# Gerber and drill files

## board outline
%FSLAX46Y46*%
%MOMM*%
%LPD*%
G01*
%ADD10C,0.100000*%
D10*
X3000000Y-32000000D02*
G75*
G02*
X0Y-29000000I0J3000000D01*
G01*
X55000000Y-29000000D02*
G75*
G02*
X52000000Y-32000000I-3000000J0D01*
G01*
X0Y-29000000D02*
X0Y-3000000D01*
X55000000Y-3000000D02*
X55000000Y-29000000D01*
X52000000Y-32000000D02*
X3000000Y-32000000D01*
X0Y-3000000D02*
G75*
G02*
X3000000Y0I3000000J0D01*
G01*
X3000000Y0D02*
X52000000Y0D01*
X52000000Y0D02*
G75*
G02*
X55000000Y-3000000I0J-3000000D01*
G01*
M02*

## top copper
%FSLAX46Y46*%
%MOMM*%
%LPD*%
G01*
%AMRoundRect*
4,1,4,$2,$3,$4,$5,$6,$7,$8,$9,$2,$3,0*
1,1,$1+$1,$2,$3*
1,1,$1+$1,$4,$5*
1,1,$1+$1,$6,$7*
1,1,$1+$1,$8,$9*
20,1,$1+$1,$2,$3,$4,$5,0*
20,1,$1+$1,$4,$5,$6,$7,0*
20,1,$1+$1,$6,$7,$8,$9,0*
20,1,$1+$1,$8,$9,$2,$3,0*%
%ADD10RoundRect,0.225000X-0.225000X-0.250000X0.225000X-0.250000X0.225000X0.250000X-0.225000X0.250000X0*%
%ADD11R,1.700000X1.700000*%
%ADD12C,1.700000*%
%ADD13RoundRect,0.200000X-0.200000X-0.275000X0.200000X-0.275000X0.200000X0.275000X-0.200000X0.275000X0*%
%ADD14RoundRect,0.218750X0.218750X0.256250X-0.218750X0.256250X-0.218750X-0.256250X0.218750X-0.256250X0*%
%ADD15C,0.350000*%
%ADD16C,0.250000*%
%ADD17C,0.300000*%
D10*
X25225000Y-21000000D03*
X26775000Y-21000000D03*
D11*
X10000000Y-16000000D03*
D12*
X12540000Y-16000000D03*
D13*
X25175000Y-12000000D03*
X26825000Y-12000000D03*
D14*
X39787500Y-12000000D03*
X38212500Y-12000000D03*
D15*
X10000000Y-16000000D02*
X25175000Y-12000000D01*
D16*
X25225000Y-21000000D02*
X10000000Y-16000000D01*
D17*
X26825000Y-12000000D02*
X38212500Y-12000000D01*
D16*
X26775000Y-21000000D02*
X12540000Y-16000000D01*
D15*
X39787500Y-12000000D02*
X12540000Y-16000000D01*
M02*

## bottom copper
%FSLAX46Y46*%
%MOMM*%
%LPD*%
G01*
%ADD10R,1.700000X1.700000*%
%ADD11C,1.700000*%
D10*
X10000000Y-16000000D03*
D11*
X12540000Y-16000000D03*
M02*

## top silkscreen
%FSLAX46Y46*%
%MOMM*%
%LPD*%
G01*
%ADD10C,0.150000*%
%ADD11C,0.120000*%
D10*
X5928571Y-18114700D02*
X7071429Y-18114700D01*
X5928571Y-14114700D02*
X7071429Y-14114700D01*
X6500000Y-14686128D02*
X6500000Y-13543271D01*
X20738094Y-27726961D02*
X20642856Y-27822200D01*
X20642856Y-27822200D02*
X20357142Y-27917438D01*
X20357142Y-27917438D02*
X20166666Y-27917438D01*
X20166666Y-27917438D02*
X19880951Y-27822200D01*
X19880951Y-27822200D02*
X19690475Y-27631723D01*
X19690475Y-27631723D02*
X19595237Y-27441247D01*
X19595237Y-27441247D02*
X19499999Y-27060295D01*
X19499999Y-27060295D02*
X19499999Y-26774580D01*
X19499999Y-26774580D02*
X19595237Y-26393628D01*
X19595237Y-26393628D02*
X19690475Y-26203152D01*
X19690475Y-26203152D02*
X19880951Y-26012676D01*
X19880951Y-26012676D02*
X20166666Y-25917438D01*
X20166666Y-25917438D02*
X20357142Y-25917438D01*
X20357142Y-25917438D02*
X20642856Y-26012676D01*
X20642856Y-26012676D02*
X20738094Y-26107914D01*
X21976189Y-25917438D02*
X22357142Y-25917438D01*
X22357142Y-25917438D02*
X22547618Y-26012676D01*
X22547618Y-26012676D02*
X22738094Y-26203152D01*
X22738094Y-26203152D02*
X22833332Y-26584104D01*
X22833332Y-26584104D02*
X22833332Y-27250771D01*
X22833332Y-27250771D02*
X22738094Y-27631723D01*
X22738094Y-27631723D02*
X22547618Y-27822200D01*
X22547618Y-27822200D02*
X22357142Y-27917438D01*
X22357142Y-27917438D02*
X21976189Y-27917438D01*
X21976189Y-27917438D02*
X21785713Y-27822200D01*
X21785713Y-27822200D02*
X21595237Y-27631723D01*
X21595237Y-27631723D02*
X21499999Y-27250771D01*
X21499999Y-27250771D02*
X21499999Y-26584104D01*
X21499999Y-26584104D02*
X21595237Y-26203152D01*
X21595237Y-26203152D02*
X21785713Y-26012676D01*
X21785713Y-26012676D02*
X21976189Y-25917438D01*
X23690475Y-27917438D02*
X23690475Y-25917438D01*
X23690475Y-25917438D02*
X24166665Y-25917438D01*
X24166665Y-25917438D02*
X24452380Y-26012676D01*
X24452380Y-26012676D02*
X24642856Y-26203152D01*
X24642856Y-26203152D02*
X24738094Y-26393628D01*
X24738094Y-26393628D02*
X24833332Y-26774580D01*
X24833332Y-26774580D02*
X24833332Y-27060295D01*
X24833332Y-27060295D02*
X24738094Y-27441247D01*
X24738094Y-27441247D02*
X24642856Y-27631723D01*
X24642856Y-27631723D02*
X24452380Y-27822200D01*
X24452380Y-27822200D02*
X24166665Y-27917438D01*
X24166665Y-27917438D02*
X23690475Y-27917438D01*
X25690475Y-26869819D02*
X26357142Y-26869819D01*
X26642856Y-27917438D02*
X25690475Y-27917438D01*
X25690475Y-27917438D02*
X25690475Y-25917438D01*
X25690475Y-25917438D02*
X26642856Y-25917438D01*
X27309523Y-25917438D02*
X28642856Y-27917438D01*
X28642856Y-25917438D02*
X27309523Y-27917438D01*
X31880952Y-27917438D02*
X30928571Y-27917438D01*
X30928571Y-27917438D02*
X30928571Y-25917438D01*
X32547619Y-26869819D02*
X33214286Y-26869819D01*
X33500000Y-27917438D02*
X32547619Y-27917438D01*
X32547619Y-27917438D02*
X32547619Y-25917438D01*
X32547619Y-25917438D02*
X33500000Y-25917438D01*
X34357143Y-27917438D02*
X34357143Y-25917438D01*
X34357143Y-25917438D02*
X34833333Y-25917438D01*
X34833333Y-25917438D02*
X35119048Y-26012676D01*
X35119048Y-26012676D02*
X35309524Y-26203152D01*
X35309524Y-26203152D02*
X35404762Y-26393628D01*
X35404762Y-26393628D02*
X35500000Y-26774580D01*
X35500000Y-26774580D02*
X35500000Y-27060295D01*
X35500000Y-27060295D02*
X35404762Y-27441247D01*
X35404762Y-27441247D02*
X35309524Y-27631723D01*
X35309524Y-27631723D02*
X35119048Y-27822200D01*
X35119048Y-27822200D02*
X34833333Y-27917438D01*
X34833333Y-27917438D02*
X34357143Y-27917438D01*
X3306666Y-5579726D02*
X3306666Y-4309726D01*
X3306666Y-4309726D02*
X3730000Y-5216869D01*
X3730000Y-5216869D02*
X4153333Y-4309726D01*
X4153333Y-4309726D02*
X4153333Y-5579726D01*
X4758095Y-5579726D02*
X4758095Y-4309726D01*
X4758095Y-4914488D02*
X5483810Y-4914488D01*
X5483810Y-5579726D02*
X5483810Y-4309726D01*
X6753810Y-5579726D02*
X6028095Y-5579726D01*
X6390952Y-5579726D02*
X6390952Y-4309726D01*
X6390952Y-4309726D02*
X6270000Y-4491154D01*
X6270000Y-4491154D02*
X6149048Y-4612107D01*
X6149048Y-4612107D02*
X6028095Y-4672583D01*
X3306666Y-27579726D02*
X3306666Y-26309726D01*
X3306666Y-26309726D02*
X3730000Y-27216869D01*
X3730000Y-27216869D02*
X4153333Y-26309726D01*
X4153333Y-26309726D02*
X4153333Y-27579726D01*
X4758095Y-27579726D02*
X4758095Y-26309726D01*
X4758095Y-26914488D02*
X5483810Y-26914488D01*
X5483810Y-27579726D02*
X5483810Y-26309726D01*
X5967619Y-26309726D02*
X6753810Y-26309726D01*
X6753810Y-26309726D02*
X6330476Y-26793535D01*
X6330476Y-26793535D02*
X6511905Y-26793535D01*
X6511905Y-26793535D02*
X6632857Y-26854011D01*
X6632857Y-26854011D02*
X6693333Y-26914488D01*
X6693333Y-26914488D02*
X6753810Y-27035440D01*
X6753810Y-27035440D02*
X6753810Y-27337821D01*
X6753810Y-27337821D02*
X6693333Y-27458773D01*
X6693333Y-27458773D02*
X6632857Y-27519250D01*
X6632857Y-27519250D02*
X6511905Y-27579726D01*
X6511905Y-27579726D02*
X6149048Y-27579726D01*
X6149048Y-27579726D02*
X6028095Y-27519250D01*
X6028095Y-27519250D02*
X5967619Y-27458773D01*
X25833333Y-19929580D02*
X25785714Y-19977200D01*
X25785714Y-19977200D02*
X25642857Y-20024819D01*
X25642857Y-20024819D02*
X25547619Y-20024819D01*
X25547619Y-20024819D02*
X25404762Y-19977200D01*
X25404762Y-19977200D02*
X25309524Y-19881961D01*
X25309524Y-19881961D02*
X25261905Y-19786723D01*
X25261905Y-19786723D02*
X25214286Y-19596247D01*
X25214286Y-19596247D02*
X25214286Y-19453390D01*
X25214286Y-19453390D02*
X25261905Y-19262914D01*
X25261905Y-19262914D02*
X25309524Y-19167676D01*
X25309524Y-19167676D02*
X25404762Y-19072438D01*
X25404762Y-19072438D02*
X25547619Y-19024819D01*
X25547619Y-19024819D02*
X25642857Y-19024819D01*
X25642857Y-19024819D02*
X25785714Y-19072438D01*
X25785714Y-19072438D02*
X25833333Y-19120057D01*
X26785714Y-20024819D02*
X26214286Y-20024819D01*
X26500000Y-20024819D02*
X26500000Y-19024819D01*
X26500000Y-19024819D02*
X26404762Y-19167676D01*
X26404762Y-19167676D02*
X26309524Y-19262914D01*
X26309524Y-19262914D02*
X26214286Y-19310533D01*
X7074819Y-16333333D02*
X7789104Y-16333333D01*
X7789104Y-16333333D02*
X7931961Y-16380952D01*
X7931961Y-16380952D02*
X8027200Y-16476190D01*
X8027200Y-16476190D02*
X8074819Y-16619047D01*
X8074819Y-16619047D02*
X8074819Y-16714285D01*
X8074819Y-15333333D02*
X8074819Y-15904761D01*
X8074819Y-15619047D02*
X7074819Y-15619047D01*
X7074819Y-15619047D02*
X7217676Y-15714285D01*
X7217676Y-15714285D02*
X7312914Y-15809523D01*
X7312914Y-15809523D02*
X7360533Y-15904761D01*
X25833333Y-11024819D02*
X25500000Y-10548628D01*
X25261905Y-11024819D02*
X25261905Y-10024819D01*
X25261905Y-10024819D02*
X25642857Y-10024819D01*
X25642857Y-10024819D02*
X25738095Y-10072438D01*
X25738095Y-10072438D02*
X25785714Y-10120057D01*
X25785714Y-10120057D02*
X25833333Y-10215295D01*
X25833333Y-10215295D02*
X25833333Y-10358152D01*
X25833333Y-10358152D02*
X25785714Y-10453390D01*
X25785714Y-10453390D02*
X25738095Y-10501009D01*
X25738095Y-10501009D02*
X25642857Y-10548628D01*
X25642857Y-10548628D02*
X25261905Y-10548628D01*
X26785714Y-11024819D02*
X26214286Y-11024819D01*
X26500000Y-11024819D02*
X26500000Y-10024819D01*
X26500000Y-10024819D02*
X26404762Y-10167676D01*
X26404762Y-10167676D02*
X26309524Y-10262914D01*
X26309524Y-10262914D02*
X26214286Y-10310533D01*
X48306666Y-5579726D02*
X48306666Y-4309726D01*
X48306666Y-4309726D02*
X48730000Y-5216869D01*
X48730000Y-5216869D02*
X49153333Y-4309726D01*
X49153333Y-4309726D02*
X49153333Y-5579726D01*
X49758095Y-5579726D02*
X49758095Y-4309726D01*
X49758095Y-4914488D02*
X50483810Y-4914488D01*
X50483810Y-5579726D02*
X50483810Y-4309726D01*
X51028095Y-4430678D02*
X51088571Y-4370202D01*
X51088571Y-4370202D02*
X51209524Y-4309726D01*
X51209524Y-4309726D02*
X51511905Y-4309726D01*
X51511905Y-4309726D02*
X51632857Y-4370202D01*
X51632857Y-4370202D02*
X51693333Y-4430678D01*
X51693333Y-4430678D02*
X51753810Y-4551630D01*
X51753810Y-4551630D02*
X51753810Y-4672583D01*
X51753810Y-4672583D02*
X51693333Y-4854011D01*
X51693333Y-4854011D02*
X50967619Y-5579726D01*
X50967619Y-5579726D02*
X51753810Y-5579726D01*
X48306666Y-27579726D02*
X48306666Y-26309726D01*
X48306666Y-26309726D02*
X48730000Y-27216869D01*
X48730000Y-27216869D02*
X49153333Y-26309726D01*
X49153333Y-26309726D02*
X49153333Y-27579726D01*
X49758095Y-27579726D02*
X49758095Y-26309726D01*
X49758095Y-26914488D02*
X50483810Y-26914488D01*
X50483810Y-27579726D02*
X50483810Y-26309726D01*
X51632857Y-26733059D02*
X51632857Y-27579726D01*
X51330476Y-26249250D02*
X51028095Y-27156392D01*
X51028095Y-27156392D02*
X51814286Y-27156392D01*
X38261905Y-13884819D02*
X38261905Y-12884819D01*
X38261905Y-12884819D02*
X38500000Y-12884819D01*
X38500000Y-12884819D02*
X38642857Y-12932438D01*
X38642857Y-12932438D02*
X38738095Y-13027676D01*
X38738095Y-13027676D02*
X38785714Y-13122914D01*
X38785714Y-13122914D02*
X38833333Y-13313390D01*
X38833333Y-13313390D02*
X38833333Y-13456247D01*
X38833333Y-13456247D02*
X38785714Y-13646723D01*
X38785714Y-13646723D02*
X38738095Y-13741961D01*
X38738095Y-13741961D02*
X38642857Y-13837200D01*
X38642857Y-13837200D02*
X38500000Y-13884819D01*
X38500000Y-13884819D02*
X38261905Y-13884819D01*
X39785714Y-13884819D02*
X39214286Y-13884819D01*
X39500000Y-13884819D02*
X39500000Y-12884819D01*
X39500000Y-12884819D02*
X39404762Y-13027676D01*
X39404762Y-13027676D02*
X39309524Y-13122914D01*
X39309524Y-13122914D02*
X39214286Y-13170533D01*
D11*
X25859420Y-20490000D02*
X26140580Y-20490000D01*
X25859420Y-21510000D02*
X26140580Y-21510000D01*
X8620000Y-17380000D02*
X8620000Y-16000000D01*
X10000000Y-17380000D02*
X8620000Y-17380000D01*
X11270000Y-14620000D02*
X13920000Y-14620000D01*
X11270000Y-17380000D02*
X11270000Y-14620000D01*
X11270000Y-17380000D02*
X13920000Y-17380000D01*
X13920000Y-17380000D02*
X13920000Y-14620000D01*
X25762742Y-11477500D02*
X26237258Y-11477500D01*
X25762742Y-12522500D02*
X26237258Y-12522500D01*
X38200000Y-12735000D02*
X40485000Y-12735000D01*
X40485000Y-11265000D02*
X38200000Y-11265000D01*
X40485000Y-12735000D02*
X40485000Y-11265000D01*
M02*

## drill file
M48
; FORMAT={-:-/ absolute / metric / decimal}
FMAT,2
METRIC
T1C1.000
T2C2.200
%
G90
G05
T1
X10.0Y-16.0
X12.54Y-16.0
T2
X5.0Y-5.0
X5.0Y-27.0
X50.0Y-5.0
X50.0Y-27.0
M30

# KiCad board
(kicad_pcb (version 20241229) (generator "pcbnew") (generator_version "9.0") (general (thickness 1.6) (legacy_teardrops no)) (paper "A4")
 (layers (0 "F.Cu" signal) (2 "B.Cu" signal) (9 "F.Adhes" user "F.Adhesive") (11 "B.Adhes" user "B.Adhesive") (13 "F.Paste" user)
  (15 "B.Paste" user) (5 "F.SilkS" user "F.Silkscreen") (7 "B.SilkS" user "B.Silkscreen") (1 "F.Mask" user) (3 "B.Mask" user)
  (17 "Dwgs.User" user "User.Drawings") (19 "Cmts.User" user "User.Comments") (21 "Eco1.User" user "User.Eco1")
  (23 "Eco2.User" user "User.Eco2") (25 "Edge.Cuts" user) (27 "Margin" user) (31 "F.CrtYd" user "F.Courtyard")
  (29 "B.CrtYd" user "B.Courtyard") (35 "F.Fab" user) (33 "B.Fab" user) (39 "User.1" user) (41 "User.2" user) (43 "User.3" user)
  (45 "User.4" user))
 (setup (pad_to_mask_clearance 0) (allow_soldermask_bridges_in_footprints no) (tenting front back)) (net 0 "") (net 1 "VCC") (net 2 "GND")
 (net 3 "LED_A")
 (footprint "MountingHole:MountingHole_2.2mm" (layer "F.Cu") (at 5 5)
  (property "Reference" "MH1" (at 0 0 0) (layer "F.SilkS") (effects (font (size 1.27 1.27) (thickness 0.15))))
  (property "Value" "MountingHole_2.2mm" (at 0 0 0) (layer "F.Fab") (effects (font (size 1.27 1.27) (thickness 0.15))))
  (pad "" np_thru_hole circle (at 0 0) (size 3.2 3.2) (drill 2.2) (layers "*.Mask")))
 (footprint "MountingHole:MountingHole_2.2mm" (layer "F.Cu") (at 5 27)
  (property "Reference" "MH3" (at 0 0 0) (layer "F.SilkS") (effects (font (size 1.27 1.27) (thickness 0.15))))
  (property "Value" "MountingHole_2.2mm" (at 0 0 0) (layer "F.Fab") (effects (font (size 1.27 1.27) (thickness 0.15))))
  (pad "" np_thru_hole circle (at 0 0) (size 3.2 3.2) (drill 2.2) (layers "*.Mask")))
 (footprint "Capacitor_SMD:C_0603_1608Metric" (layer "F.Cu") (at 26 21)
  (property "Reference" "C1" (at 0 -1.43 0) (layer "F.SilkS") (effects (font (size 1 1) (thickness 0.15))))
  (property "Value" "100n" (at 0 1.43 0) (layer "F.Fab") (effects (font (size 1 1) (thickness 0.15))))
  (fp_line (start -0.14058 -0.51) (end 0.14058 -0.51) (stroke (width 0.12) (type solid)) (layer "F.SilkS"))
  (fp_line (start -0.14058 0.51) (end 0.14058 0.51) (stroke (width 0.12) (type solid)) (layer "F.SilkS"))
  (pad "1" smd roundrect (at -0.775 0) (size 0.9 0.95) (layers "F.Cu" "F.Mask" "F.Paste") (roundrect_rratio 0.25) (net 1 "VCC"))
  (pad "2" smd roundrect (at 0.775 0) (size 0.9 0.95) (layers "F.Cu" "F.Mask" "F.Paste") (roundrect_rratio 0.25) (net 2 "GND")))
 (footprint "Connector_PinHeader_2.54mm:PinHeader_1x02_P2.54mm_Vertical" (layer "F.Cu") (at 10 16 90)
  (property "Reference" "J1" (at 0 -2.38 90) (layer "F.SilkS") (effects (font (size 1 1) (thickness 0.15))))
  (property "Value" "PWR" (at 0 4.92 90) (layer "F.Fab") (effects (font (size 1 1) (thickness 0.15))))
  (fp_line (start -1.38 -1.38) (end 0 -1.38) (stroke (width 0.12) (type solid)) (layer "F.SilkS"))
  (fp_line (start -1.38 0) (end -1.38 -1.38) (stroke (width 0.12) (type solid)) (layer "F.SilkS"))
  (fp_line (start 1.38 1.27) (end 1.38 3.92) (stroke (width 0.12) (type solid)) (layer "F.SilkS"))
  (fp_line (start -1.38 1.27) (end 1.38 1.27) (stroke (width 0.12) (type solid)) (layer "F.SilkS"))
  (fp_line (start -1.38 1.27) (end -1.38 3.92) (stroke (width 0.12) (type solid)) (layer "F.SilkS"))
  (fp_line (start -1.38 3.92) (end 1.38 3.92) (stroke (width 0.12) (type solid)) (layer "F.SilkS"))
  (pad "1" thru_hole rect (at 0 0 90) (size 1.7 1.7) (drill 1) (layers "*.Cu" "*.Mask") (remove_unused_layers no) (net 1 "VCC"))
  (pad "2" thru_hole circle (at 0 2.54 90) (size 1.7 1.7) (drill 1) (layers "*.Cu" "*.Mask") (remove_unused_layers no) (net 2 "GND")))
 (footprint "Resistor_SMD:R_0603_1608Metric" (layer "F.Cu") (at 26 12)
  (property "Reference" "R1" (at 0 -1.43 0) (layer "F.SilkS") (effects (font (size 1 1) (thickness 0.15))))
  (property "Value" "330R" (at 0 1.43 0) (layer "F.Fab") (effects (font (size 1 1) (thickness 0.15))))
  (fp_line (start -0.237258 -0.5225) (end 0.237258 -0.5225) (stroke (width 0.12) (type solid)) (layer "F.SilkS"))
  (fp_line (start -0.237258 0.5225) (end 0.237258 0.5225) (stroke (width 0.12) (type solid)) (layer "F.SilkS"))
  (pad "1" smd roundrect (at -0.825 0) (size 0.8 0.95) (layers "F.Cu" "F.Mask" "F.Paste") (roundrect_rratio 0.25) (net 1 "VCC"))
  (pad "2" smd roundrect (at 0.825 0) (size 0.8 0.95) (layers "F.Cu" "F.Mask" "F.Paste") (roundrect_rratio 0.25) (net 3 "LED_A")))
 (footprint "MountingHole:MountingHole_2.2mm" (layer "F.Cu") (at 50 5)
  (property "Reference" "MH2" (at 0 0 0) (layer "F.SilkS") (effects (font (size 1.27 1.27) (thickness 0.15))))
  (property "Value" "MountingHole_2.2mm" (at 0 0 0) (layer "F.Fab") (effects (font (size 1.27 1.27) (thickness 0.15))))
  (pad "" np_thru_hole circle (at 0 0) (size 3.2 3.2) (drill 2.2) (layers "*.Mask")))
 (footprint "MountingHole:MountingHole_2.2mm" (layer "F.Cu") (at 50 27)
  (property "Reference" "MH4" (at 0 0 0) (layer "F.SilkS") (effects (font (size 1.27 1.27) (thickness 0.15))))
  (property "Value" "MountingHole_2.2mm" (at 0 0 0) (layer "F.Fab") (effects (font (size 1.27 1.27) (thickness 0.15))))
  (pad "" np_thru_hole circle (at 0 0) (size 3.2 3.2) (drill 2.2) (layers "*.Mask")))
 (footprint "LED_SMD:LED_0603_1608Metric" (layer "F.Cu") (at 39 12 180)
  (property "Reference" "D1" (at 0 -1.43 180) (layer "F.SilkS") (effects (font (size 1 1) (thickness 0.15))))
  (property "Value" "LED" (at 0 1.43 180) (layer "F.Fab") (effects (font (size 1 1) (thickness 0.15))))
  (fp_line (start 0.8 -0.735) (end -1.485 -0.735) (stroke (width 0.12) (type solid)) (layer "F.SilkS"))
  (fp_line (start -1.485 0.735) (end 0.8 0.735) (stroke (width 0.12) (type solid)) (layer "F.SilkS"))
  (fp_line (start -1.485 -0.735) (end -1.485 0.735) (stroke (width 0.12) (type solid)) (layer "F.SilkS"))
  (pad "1" smd roundrect (at -0.7875 0 180) (size 0.875 0.95) (layers "F.Cu" "F.Mask" "F.Paste") (roundrect_rratio 0.25) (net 2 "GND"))
  (pad "2" smd roundrect (at 0.7875 0 180) (size 0.875 0.95) (layers "F.Cu" "F.Mask" "F.Paste") (roundrect_rratio 0.25) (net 3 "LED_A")))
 (gr_arc (start 3 32) (mid 0.87868 31.12132) (end 0 29) (stroke (width 0.1) (type default)) (layer "Edge.Cuts"))
 (gr_arc (start 55 29) (mid 54.12132 31.12132) (end 52 32) (stroke (width 0.1) (type default)) (layer "Edge.Cuts"))
 (gr_line (start 0 29) (end 0 3) (stroke (width 0.1) (type default)) (layer "Edge.Cuts"))
 (gr_line (start 55 3) (end 55 29) (stroke (width 0.1) (type default)) (layer "Edge.Cuts"))
 (gr_line (start 52 32) (end 3 32) (stroke (width 0.1) (type default)) (layer "Edge.Cuts"))
 (gr_arc (start 0 3) (mid 0.87868 0.87868) (end 3 0) (stroke (width 0.1) (type default)) (layer "Edge.Cuts"))
 (gr_line (start 3 0) (end 52 0) (stroke (width 0.1) (type default)) (layer "Edge.Cuts"))
 (gr_arc (start 52 0) (mid 54.12132 0.87868) (end 55 3) (stroke (width 0.1) (type default)) (layer "Edge.Cuts"))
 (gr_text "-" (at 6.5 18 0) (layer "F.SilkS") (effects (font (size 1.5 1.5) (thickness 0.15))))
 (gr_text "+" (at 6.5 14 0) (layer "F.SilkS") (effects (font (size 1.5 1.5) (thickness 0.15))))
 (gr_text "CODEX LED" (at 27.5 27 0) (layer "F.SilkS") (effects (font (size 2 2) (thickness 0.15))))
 (segment (start 10 16) (end 25.175 12) (width 0.35) (layer "F.Cu") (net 1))
 (segment (start 25.225 21) (end 10 16) (width 0.25) (layer "F.Cu") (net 1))
 (segment (start 26.825 12) (end 38.2125 12) (width 0.3) (layer "F.Cu") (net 3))
 (segment (start 26.775 21) (end 12.54 16) (width 0.25) (layer "F.Cu") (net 2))
 (segment (start 39.7875 12) (end 12.54 16) (width 0.35) (layer "F.Cu") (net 2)))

